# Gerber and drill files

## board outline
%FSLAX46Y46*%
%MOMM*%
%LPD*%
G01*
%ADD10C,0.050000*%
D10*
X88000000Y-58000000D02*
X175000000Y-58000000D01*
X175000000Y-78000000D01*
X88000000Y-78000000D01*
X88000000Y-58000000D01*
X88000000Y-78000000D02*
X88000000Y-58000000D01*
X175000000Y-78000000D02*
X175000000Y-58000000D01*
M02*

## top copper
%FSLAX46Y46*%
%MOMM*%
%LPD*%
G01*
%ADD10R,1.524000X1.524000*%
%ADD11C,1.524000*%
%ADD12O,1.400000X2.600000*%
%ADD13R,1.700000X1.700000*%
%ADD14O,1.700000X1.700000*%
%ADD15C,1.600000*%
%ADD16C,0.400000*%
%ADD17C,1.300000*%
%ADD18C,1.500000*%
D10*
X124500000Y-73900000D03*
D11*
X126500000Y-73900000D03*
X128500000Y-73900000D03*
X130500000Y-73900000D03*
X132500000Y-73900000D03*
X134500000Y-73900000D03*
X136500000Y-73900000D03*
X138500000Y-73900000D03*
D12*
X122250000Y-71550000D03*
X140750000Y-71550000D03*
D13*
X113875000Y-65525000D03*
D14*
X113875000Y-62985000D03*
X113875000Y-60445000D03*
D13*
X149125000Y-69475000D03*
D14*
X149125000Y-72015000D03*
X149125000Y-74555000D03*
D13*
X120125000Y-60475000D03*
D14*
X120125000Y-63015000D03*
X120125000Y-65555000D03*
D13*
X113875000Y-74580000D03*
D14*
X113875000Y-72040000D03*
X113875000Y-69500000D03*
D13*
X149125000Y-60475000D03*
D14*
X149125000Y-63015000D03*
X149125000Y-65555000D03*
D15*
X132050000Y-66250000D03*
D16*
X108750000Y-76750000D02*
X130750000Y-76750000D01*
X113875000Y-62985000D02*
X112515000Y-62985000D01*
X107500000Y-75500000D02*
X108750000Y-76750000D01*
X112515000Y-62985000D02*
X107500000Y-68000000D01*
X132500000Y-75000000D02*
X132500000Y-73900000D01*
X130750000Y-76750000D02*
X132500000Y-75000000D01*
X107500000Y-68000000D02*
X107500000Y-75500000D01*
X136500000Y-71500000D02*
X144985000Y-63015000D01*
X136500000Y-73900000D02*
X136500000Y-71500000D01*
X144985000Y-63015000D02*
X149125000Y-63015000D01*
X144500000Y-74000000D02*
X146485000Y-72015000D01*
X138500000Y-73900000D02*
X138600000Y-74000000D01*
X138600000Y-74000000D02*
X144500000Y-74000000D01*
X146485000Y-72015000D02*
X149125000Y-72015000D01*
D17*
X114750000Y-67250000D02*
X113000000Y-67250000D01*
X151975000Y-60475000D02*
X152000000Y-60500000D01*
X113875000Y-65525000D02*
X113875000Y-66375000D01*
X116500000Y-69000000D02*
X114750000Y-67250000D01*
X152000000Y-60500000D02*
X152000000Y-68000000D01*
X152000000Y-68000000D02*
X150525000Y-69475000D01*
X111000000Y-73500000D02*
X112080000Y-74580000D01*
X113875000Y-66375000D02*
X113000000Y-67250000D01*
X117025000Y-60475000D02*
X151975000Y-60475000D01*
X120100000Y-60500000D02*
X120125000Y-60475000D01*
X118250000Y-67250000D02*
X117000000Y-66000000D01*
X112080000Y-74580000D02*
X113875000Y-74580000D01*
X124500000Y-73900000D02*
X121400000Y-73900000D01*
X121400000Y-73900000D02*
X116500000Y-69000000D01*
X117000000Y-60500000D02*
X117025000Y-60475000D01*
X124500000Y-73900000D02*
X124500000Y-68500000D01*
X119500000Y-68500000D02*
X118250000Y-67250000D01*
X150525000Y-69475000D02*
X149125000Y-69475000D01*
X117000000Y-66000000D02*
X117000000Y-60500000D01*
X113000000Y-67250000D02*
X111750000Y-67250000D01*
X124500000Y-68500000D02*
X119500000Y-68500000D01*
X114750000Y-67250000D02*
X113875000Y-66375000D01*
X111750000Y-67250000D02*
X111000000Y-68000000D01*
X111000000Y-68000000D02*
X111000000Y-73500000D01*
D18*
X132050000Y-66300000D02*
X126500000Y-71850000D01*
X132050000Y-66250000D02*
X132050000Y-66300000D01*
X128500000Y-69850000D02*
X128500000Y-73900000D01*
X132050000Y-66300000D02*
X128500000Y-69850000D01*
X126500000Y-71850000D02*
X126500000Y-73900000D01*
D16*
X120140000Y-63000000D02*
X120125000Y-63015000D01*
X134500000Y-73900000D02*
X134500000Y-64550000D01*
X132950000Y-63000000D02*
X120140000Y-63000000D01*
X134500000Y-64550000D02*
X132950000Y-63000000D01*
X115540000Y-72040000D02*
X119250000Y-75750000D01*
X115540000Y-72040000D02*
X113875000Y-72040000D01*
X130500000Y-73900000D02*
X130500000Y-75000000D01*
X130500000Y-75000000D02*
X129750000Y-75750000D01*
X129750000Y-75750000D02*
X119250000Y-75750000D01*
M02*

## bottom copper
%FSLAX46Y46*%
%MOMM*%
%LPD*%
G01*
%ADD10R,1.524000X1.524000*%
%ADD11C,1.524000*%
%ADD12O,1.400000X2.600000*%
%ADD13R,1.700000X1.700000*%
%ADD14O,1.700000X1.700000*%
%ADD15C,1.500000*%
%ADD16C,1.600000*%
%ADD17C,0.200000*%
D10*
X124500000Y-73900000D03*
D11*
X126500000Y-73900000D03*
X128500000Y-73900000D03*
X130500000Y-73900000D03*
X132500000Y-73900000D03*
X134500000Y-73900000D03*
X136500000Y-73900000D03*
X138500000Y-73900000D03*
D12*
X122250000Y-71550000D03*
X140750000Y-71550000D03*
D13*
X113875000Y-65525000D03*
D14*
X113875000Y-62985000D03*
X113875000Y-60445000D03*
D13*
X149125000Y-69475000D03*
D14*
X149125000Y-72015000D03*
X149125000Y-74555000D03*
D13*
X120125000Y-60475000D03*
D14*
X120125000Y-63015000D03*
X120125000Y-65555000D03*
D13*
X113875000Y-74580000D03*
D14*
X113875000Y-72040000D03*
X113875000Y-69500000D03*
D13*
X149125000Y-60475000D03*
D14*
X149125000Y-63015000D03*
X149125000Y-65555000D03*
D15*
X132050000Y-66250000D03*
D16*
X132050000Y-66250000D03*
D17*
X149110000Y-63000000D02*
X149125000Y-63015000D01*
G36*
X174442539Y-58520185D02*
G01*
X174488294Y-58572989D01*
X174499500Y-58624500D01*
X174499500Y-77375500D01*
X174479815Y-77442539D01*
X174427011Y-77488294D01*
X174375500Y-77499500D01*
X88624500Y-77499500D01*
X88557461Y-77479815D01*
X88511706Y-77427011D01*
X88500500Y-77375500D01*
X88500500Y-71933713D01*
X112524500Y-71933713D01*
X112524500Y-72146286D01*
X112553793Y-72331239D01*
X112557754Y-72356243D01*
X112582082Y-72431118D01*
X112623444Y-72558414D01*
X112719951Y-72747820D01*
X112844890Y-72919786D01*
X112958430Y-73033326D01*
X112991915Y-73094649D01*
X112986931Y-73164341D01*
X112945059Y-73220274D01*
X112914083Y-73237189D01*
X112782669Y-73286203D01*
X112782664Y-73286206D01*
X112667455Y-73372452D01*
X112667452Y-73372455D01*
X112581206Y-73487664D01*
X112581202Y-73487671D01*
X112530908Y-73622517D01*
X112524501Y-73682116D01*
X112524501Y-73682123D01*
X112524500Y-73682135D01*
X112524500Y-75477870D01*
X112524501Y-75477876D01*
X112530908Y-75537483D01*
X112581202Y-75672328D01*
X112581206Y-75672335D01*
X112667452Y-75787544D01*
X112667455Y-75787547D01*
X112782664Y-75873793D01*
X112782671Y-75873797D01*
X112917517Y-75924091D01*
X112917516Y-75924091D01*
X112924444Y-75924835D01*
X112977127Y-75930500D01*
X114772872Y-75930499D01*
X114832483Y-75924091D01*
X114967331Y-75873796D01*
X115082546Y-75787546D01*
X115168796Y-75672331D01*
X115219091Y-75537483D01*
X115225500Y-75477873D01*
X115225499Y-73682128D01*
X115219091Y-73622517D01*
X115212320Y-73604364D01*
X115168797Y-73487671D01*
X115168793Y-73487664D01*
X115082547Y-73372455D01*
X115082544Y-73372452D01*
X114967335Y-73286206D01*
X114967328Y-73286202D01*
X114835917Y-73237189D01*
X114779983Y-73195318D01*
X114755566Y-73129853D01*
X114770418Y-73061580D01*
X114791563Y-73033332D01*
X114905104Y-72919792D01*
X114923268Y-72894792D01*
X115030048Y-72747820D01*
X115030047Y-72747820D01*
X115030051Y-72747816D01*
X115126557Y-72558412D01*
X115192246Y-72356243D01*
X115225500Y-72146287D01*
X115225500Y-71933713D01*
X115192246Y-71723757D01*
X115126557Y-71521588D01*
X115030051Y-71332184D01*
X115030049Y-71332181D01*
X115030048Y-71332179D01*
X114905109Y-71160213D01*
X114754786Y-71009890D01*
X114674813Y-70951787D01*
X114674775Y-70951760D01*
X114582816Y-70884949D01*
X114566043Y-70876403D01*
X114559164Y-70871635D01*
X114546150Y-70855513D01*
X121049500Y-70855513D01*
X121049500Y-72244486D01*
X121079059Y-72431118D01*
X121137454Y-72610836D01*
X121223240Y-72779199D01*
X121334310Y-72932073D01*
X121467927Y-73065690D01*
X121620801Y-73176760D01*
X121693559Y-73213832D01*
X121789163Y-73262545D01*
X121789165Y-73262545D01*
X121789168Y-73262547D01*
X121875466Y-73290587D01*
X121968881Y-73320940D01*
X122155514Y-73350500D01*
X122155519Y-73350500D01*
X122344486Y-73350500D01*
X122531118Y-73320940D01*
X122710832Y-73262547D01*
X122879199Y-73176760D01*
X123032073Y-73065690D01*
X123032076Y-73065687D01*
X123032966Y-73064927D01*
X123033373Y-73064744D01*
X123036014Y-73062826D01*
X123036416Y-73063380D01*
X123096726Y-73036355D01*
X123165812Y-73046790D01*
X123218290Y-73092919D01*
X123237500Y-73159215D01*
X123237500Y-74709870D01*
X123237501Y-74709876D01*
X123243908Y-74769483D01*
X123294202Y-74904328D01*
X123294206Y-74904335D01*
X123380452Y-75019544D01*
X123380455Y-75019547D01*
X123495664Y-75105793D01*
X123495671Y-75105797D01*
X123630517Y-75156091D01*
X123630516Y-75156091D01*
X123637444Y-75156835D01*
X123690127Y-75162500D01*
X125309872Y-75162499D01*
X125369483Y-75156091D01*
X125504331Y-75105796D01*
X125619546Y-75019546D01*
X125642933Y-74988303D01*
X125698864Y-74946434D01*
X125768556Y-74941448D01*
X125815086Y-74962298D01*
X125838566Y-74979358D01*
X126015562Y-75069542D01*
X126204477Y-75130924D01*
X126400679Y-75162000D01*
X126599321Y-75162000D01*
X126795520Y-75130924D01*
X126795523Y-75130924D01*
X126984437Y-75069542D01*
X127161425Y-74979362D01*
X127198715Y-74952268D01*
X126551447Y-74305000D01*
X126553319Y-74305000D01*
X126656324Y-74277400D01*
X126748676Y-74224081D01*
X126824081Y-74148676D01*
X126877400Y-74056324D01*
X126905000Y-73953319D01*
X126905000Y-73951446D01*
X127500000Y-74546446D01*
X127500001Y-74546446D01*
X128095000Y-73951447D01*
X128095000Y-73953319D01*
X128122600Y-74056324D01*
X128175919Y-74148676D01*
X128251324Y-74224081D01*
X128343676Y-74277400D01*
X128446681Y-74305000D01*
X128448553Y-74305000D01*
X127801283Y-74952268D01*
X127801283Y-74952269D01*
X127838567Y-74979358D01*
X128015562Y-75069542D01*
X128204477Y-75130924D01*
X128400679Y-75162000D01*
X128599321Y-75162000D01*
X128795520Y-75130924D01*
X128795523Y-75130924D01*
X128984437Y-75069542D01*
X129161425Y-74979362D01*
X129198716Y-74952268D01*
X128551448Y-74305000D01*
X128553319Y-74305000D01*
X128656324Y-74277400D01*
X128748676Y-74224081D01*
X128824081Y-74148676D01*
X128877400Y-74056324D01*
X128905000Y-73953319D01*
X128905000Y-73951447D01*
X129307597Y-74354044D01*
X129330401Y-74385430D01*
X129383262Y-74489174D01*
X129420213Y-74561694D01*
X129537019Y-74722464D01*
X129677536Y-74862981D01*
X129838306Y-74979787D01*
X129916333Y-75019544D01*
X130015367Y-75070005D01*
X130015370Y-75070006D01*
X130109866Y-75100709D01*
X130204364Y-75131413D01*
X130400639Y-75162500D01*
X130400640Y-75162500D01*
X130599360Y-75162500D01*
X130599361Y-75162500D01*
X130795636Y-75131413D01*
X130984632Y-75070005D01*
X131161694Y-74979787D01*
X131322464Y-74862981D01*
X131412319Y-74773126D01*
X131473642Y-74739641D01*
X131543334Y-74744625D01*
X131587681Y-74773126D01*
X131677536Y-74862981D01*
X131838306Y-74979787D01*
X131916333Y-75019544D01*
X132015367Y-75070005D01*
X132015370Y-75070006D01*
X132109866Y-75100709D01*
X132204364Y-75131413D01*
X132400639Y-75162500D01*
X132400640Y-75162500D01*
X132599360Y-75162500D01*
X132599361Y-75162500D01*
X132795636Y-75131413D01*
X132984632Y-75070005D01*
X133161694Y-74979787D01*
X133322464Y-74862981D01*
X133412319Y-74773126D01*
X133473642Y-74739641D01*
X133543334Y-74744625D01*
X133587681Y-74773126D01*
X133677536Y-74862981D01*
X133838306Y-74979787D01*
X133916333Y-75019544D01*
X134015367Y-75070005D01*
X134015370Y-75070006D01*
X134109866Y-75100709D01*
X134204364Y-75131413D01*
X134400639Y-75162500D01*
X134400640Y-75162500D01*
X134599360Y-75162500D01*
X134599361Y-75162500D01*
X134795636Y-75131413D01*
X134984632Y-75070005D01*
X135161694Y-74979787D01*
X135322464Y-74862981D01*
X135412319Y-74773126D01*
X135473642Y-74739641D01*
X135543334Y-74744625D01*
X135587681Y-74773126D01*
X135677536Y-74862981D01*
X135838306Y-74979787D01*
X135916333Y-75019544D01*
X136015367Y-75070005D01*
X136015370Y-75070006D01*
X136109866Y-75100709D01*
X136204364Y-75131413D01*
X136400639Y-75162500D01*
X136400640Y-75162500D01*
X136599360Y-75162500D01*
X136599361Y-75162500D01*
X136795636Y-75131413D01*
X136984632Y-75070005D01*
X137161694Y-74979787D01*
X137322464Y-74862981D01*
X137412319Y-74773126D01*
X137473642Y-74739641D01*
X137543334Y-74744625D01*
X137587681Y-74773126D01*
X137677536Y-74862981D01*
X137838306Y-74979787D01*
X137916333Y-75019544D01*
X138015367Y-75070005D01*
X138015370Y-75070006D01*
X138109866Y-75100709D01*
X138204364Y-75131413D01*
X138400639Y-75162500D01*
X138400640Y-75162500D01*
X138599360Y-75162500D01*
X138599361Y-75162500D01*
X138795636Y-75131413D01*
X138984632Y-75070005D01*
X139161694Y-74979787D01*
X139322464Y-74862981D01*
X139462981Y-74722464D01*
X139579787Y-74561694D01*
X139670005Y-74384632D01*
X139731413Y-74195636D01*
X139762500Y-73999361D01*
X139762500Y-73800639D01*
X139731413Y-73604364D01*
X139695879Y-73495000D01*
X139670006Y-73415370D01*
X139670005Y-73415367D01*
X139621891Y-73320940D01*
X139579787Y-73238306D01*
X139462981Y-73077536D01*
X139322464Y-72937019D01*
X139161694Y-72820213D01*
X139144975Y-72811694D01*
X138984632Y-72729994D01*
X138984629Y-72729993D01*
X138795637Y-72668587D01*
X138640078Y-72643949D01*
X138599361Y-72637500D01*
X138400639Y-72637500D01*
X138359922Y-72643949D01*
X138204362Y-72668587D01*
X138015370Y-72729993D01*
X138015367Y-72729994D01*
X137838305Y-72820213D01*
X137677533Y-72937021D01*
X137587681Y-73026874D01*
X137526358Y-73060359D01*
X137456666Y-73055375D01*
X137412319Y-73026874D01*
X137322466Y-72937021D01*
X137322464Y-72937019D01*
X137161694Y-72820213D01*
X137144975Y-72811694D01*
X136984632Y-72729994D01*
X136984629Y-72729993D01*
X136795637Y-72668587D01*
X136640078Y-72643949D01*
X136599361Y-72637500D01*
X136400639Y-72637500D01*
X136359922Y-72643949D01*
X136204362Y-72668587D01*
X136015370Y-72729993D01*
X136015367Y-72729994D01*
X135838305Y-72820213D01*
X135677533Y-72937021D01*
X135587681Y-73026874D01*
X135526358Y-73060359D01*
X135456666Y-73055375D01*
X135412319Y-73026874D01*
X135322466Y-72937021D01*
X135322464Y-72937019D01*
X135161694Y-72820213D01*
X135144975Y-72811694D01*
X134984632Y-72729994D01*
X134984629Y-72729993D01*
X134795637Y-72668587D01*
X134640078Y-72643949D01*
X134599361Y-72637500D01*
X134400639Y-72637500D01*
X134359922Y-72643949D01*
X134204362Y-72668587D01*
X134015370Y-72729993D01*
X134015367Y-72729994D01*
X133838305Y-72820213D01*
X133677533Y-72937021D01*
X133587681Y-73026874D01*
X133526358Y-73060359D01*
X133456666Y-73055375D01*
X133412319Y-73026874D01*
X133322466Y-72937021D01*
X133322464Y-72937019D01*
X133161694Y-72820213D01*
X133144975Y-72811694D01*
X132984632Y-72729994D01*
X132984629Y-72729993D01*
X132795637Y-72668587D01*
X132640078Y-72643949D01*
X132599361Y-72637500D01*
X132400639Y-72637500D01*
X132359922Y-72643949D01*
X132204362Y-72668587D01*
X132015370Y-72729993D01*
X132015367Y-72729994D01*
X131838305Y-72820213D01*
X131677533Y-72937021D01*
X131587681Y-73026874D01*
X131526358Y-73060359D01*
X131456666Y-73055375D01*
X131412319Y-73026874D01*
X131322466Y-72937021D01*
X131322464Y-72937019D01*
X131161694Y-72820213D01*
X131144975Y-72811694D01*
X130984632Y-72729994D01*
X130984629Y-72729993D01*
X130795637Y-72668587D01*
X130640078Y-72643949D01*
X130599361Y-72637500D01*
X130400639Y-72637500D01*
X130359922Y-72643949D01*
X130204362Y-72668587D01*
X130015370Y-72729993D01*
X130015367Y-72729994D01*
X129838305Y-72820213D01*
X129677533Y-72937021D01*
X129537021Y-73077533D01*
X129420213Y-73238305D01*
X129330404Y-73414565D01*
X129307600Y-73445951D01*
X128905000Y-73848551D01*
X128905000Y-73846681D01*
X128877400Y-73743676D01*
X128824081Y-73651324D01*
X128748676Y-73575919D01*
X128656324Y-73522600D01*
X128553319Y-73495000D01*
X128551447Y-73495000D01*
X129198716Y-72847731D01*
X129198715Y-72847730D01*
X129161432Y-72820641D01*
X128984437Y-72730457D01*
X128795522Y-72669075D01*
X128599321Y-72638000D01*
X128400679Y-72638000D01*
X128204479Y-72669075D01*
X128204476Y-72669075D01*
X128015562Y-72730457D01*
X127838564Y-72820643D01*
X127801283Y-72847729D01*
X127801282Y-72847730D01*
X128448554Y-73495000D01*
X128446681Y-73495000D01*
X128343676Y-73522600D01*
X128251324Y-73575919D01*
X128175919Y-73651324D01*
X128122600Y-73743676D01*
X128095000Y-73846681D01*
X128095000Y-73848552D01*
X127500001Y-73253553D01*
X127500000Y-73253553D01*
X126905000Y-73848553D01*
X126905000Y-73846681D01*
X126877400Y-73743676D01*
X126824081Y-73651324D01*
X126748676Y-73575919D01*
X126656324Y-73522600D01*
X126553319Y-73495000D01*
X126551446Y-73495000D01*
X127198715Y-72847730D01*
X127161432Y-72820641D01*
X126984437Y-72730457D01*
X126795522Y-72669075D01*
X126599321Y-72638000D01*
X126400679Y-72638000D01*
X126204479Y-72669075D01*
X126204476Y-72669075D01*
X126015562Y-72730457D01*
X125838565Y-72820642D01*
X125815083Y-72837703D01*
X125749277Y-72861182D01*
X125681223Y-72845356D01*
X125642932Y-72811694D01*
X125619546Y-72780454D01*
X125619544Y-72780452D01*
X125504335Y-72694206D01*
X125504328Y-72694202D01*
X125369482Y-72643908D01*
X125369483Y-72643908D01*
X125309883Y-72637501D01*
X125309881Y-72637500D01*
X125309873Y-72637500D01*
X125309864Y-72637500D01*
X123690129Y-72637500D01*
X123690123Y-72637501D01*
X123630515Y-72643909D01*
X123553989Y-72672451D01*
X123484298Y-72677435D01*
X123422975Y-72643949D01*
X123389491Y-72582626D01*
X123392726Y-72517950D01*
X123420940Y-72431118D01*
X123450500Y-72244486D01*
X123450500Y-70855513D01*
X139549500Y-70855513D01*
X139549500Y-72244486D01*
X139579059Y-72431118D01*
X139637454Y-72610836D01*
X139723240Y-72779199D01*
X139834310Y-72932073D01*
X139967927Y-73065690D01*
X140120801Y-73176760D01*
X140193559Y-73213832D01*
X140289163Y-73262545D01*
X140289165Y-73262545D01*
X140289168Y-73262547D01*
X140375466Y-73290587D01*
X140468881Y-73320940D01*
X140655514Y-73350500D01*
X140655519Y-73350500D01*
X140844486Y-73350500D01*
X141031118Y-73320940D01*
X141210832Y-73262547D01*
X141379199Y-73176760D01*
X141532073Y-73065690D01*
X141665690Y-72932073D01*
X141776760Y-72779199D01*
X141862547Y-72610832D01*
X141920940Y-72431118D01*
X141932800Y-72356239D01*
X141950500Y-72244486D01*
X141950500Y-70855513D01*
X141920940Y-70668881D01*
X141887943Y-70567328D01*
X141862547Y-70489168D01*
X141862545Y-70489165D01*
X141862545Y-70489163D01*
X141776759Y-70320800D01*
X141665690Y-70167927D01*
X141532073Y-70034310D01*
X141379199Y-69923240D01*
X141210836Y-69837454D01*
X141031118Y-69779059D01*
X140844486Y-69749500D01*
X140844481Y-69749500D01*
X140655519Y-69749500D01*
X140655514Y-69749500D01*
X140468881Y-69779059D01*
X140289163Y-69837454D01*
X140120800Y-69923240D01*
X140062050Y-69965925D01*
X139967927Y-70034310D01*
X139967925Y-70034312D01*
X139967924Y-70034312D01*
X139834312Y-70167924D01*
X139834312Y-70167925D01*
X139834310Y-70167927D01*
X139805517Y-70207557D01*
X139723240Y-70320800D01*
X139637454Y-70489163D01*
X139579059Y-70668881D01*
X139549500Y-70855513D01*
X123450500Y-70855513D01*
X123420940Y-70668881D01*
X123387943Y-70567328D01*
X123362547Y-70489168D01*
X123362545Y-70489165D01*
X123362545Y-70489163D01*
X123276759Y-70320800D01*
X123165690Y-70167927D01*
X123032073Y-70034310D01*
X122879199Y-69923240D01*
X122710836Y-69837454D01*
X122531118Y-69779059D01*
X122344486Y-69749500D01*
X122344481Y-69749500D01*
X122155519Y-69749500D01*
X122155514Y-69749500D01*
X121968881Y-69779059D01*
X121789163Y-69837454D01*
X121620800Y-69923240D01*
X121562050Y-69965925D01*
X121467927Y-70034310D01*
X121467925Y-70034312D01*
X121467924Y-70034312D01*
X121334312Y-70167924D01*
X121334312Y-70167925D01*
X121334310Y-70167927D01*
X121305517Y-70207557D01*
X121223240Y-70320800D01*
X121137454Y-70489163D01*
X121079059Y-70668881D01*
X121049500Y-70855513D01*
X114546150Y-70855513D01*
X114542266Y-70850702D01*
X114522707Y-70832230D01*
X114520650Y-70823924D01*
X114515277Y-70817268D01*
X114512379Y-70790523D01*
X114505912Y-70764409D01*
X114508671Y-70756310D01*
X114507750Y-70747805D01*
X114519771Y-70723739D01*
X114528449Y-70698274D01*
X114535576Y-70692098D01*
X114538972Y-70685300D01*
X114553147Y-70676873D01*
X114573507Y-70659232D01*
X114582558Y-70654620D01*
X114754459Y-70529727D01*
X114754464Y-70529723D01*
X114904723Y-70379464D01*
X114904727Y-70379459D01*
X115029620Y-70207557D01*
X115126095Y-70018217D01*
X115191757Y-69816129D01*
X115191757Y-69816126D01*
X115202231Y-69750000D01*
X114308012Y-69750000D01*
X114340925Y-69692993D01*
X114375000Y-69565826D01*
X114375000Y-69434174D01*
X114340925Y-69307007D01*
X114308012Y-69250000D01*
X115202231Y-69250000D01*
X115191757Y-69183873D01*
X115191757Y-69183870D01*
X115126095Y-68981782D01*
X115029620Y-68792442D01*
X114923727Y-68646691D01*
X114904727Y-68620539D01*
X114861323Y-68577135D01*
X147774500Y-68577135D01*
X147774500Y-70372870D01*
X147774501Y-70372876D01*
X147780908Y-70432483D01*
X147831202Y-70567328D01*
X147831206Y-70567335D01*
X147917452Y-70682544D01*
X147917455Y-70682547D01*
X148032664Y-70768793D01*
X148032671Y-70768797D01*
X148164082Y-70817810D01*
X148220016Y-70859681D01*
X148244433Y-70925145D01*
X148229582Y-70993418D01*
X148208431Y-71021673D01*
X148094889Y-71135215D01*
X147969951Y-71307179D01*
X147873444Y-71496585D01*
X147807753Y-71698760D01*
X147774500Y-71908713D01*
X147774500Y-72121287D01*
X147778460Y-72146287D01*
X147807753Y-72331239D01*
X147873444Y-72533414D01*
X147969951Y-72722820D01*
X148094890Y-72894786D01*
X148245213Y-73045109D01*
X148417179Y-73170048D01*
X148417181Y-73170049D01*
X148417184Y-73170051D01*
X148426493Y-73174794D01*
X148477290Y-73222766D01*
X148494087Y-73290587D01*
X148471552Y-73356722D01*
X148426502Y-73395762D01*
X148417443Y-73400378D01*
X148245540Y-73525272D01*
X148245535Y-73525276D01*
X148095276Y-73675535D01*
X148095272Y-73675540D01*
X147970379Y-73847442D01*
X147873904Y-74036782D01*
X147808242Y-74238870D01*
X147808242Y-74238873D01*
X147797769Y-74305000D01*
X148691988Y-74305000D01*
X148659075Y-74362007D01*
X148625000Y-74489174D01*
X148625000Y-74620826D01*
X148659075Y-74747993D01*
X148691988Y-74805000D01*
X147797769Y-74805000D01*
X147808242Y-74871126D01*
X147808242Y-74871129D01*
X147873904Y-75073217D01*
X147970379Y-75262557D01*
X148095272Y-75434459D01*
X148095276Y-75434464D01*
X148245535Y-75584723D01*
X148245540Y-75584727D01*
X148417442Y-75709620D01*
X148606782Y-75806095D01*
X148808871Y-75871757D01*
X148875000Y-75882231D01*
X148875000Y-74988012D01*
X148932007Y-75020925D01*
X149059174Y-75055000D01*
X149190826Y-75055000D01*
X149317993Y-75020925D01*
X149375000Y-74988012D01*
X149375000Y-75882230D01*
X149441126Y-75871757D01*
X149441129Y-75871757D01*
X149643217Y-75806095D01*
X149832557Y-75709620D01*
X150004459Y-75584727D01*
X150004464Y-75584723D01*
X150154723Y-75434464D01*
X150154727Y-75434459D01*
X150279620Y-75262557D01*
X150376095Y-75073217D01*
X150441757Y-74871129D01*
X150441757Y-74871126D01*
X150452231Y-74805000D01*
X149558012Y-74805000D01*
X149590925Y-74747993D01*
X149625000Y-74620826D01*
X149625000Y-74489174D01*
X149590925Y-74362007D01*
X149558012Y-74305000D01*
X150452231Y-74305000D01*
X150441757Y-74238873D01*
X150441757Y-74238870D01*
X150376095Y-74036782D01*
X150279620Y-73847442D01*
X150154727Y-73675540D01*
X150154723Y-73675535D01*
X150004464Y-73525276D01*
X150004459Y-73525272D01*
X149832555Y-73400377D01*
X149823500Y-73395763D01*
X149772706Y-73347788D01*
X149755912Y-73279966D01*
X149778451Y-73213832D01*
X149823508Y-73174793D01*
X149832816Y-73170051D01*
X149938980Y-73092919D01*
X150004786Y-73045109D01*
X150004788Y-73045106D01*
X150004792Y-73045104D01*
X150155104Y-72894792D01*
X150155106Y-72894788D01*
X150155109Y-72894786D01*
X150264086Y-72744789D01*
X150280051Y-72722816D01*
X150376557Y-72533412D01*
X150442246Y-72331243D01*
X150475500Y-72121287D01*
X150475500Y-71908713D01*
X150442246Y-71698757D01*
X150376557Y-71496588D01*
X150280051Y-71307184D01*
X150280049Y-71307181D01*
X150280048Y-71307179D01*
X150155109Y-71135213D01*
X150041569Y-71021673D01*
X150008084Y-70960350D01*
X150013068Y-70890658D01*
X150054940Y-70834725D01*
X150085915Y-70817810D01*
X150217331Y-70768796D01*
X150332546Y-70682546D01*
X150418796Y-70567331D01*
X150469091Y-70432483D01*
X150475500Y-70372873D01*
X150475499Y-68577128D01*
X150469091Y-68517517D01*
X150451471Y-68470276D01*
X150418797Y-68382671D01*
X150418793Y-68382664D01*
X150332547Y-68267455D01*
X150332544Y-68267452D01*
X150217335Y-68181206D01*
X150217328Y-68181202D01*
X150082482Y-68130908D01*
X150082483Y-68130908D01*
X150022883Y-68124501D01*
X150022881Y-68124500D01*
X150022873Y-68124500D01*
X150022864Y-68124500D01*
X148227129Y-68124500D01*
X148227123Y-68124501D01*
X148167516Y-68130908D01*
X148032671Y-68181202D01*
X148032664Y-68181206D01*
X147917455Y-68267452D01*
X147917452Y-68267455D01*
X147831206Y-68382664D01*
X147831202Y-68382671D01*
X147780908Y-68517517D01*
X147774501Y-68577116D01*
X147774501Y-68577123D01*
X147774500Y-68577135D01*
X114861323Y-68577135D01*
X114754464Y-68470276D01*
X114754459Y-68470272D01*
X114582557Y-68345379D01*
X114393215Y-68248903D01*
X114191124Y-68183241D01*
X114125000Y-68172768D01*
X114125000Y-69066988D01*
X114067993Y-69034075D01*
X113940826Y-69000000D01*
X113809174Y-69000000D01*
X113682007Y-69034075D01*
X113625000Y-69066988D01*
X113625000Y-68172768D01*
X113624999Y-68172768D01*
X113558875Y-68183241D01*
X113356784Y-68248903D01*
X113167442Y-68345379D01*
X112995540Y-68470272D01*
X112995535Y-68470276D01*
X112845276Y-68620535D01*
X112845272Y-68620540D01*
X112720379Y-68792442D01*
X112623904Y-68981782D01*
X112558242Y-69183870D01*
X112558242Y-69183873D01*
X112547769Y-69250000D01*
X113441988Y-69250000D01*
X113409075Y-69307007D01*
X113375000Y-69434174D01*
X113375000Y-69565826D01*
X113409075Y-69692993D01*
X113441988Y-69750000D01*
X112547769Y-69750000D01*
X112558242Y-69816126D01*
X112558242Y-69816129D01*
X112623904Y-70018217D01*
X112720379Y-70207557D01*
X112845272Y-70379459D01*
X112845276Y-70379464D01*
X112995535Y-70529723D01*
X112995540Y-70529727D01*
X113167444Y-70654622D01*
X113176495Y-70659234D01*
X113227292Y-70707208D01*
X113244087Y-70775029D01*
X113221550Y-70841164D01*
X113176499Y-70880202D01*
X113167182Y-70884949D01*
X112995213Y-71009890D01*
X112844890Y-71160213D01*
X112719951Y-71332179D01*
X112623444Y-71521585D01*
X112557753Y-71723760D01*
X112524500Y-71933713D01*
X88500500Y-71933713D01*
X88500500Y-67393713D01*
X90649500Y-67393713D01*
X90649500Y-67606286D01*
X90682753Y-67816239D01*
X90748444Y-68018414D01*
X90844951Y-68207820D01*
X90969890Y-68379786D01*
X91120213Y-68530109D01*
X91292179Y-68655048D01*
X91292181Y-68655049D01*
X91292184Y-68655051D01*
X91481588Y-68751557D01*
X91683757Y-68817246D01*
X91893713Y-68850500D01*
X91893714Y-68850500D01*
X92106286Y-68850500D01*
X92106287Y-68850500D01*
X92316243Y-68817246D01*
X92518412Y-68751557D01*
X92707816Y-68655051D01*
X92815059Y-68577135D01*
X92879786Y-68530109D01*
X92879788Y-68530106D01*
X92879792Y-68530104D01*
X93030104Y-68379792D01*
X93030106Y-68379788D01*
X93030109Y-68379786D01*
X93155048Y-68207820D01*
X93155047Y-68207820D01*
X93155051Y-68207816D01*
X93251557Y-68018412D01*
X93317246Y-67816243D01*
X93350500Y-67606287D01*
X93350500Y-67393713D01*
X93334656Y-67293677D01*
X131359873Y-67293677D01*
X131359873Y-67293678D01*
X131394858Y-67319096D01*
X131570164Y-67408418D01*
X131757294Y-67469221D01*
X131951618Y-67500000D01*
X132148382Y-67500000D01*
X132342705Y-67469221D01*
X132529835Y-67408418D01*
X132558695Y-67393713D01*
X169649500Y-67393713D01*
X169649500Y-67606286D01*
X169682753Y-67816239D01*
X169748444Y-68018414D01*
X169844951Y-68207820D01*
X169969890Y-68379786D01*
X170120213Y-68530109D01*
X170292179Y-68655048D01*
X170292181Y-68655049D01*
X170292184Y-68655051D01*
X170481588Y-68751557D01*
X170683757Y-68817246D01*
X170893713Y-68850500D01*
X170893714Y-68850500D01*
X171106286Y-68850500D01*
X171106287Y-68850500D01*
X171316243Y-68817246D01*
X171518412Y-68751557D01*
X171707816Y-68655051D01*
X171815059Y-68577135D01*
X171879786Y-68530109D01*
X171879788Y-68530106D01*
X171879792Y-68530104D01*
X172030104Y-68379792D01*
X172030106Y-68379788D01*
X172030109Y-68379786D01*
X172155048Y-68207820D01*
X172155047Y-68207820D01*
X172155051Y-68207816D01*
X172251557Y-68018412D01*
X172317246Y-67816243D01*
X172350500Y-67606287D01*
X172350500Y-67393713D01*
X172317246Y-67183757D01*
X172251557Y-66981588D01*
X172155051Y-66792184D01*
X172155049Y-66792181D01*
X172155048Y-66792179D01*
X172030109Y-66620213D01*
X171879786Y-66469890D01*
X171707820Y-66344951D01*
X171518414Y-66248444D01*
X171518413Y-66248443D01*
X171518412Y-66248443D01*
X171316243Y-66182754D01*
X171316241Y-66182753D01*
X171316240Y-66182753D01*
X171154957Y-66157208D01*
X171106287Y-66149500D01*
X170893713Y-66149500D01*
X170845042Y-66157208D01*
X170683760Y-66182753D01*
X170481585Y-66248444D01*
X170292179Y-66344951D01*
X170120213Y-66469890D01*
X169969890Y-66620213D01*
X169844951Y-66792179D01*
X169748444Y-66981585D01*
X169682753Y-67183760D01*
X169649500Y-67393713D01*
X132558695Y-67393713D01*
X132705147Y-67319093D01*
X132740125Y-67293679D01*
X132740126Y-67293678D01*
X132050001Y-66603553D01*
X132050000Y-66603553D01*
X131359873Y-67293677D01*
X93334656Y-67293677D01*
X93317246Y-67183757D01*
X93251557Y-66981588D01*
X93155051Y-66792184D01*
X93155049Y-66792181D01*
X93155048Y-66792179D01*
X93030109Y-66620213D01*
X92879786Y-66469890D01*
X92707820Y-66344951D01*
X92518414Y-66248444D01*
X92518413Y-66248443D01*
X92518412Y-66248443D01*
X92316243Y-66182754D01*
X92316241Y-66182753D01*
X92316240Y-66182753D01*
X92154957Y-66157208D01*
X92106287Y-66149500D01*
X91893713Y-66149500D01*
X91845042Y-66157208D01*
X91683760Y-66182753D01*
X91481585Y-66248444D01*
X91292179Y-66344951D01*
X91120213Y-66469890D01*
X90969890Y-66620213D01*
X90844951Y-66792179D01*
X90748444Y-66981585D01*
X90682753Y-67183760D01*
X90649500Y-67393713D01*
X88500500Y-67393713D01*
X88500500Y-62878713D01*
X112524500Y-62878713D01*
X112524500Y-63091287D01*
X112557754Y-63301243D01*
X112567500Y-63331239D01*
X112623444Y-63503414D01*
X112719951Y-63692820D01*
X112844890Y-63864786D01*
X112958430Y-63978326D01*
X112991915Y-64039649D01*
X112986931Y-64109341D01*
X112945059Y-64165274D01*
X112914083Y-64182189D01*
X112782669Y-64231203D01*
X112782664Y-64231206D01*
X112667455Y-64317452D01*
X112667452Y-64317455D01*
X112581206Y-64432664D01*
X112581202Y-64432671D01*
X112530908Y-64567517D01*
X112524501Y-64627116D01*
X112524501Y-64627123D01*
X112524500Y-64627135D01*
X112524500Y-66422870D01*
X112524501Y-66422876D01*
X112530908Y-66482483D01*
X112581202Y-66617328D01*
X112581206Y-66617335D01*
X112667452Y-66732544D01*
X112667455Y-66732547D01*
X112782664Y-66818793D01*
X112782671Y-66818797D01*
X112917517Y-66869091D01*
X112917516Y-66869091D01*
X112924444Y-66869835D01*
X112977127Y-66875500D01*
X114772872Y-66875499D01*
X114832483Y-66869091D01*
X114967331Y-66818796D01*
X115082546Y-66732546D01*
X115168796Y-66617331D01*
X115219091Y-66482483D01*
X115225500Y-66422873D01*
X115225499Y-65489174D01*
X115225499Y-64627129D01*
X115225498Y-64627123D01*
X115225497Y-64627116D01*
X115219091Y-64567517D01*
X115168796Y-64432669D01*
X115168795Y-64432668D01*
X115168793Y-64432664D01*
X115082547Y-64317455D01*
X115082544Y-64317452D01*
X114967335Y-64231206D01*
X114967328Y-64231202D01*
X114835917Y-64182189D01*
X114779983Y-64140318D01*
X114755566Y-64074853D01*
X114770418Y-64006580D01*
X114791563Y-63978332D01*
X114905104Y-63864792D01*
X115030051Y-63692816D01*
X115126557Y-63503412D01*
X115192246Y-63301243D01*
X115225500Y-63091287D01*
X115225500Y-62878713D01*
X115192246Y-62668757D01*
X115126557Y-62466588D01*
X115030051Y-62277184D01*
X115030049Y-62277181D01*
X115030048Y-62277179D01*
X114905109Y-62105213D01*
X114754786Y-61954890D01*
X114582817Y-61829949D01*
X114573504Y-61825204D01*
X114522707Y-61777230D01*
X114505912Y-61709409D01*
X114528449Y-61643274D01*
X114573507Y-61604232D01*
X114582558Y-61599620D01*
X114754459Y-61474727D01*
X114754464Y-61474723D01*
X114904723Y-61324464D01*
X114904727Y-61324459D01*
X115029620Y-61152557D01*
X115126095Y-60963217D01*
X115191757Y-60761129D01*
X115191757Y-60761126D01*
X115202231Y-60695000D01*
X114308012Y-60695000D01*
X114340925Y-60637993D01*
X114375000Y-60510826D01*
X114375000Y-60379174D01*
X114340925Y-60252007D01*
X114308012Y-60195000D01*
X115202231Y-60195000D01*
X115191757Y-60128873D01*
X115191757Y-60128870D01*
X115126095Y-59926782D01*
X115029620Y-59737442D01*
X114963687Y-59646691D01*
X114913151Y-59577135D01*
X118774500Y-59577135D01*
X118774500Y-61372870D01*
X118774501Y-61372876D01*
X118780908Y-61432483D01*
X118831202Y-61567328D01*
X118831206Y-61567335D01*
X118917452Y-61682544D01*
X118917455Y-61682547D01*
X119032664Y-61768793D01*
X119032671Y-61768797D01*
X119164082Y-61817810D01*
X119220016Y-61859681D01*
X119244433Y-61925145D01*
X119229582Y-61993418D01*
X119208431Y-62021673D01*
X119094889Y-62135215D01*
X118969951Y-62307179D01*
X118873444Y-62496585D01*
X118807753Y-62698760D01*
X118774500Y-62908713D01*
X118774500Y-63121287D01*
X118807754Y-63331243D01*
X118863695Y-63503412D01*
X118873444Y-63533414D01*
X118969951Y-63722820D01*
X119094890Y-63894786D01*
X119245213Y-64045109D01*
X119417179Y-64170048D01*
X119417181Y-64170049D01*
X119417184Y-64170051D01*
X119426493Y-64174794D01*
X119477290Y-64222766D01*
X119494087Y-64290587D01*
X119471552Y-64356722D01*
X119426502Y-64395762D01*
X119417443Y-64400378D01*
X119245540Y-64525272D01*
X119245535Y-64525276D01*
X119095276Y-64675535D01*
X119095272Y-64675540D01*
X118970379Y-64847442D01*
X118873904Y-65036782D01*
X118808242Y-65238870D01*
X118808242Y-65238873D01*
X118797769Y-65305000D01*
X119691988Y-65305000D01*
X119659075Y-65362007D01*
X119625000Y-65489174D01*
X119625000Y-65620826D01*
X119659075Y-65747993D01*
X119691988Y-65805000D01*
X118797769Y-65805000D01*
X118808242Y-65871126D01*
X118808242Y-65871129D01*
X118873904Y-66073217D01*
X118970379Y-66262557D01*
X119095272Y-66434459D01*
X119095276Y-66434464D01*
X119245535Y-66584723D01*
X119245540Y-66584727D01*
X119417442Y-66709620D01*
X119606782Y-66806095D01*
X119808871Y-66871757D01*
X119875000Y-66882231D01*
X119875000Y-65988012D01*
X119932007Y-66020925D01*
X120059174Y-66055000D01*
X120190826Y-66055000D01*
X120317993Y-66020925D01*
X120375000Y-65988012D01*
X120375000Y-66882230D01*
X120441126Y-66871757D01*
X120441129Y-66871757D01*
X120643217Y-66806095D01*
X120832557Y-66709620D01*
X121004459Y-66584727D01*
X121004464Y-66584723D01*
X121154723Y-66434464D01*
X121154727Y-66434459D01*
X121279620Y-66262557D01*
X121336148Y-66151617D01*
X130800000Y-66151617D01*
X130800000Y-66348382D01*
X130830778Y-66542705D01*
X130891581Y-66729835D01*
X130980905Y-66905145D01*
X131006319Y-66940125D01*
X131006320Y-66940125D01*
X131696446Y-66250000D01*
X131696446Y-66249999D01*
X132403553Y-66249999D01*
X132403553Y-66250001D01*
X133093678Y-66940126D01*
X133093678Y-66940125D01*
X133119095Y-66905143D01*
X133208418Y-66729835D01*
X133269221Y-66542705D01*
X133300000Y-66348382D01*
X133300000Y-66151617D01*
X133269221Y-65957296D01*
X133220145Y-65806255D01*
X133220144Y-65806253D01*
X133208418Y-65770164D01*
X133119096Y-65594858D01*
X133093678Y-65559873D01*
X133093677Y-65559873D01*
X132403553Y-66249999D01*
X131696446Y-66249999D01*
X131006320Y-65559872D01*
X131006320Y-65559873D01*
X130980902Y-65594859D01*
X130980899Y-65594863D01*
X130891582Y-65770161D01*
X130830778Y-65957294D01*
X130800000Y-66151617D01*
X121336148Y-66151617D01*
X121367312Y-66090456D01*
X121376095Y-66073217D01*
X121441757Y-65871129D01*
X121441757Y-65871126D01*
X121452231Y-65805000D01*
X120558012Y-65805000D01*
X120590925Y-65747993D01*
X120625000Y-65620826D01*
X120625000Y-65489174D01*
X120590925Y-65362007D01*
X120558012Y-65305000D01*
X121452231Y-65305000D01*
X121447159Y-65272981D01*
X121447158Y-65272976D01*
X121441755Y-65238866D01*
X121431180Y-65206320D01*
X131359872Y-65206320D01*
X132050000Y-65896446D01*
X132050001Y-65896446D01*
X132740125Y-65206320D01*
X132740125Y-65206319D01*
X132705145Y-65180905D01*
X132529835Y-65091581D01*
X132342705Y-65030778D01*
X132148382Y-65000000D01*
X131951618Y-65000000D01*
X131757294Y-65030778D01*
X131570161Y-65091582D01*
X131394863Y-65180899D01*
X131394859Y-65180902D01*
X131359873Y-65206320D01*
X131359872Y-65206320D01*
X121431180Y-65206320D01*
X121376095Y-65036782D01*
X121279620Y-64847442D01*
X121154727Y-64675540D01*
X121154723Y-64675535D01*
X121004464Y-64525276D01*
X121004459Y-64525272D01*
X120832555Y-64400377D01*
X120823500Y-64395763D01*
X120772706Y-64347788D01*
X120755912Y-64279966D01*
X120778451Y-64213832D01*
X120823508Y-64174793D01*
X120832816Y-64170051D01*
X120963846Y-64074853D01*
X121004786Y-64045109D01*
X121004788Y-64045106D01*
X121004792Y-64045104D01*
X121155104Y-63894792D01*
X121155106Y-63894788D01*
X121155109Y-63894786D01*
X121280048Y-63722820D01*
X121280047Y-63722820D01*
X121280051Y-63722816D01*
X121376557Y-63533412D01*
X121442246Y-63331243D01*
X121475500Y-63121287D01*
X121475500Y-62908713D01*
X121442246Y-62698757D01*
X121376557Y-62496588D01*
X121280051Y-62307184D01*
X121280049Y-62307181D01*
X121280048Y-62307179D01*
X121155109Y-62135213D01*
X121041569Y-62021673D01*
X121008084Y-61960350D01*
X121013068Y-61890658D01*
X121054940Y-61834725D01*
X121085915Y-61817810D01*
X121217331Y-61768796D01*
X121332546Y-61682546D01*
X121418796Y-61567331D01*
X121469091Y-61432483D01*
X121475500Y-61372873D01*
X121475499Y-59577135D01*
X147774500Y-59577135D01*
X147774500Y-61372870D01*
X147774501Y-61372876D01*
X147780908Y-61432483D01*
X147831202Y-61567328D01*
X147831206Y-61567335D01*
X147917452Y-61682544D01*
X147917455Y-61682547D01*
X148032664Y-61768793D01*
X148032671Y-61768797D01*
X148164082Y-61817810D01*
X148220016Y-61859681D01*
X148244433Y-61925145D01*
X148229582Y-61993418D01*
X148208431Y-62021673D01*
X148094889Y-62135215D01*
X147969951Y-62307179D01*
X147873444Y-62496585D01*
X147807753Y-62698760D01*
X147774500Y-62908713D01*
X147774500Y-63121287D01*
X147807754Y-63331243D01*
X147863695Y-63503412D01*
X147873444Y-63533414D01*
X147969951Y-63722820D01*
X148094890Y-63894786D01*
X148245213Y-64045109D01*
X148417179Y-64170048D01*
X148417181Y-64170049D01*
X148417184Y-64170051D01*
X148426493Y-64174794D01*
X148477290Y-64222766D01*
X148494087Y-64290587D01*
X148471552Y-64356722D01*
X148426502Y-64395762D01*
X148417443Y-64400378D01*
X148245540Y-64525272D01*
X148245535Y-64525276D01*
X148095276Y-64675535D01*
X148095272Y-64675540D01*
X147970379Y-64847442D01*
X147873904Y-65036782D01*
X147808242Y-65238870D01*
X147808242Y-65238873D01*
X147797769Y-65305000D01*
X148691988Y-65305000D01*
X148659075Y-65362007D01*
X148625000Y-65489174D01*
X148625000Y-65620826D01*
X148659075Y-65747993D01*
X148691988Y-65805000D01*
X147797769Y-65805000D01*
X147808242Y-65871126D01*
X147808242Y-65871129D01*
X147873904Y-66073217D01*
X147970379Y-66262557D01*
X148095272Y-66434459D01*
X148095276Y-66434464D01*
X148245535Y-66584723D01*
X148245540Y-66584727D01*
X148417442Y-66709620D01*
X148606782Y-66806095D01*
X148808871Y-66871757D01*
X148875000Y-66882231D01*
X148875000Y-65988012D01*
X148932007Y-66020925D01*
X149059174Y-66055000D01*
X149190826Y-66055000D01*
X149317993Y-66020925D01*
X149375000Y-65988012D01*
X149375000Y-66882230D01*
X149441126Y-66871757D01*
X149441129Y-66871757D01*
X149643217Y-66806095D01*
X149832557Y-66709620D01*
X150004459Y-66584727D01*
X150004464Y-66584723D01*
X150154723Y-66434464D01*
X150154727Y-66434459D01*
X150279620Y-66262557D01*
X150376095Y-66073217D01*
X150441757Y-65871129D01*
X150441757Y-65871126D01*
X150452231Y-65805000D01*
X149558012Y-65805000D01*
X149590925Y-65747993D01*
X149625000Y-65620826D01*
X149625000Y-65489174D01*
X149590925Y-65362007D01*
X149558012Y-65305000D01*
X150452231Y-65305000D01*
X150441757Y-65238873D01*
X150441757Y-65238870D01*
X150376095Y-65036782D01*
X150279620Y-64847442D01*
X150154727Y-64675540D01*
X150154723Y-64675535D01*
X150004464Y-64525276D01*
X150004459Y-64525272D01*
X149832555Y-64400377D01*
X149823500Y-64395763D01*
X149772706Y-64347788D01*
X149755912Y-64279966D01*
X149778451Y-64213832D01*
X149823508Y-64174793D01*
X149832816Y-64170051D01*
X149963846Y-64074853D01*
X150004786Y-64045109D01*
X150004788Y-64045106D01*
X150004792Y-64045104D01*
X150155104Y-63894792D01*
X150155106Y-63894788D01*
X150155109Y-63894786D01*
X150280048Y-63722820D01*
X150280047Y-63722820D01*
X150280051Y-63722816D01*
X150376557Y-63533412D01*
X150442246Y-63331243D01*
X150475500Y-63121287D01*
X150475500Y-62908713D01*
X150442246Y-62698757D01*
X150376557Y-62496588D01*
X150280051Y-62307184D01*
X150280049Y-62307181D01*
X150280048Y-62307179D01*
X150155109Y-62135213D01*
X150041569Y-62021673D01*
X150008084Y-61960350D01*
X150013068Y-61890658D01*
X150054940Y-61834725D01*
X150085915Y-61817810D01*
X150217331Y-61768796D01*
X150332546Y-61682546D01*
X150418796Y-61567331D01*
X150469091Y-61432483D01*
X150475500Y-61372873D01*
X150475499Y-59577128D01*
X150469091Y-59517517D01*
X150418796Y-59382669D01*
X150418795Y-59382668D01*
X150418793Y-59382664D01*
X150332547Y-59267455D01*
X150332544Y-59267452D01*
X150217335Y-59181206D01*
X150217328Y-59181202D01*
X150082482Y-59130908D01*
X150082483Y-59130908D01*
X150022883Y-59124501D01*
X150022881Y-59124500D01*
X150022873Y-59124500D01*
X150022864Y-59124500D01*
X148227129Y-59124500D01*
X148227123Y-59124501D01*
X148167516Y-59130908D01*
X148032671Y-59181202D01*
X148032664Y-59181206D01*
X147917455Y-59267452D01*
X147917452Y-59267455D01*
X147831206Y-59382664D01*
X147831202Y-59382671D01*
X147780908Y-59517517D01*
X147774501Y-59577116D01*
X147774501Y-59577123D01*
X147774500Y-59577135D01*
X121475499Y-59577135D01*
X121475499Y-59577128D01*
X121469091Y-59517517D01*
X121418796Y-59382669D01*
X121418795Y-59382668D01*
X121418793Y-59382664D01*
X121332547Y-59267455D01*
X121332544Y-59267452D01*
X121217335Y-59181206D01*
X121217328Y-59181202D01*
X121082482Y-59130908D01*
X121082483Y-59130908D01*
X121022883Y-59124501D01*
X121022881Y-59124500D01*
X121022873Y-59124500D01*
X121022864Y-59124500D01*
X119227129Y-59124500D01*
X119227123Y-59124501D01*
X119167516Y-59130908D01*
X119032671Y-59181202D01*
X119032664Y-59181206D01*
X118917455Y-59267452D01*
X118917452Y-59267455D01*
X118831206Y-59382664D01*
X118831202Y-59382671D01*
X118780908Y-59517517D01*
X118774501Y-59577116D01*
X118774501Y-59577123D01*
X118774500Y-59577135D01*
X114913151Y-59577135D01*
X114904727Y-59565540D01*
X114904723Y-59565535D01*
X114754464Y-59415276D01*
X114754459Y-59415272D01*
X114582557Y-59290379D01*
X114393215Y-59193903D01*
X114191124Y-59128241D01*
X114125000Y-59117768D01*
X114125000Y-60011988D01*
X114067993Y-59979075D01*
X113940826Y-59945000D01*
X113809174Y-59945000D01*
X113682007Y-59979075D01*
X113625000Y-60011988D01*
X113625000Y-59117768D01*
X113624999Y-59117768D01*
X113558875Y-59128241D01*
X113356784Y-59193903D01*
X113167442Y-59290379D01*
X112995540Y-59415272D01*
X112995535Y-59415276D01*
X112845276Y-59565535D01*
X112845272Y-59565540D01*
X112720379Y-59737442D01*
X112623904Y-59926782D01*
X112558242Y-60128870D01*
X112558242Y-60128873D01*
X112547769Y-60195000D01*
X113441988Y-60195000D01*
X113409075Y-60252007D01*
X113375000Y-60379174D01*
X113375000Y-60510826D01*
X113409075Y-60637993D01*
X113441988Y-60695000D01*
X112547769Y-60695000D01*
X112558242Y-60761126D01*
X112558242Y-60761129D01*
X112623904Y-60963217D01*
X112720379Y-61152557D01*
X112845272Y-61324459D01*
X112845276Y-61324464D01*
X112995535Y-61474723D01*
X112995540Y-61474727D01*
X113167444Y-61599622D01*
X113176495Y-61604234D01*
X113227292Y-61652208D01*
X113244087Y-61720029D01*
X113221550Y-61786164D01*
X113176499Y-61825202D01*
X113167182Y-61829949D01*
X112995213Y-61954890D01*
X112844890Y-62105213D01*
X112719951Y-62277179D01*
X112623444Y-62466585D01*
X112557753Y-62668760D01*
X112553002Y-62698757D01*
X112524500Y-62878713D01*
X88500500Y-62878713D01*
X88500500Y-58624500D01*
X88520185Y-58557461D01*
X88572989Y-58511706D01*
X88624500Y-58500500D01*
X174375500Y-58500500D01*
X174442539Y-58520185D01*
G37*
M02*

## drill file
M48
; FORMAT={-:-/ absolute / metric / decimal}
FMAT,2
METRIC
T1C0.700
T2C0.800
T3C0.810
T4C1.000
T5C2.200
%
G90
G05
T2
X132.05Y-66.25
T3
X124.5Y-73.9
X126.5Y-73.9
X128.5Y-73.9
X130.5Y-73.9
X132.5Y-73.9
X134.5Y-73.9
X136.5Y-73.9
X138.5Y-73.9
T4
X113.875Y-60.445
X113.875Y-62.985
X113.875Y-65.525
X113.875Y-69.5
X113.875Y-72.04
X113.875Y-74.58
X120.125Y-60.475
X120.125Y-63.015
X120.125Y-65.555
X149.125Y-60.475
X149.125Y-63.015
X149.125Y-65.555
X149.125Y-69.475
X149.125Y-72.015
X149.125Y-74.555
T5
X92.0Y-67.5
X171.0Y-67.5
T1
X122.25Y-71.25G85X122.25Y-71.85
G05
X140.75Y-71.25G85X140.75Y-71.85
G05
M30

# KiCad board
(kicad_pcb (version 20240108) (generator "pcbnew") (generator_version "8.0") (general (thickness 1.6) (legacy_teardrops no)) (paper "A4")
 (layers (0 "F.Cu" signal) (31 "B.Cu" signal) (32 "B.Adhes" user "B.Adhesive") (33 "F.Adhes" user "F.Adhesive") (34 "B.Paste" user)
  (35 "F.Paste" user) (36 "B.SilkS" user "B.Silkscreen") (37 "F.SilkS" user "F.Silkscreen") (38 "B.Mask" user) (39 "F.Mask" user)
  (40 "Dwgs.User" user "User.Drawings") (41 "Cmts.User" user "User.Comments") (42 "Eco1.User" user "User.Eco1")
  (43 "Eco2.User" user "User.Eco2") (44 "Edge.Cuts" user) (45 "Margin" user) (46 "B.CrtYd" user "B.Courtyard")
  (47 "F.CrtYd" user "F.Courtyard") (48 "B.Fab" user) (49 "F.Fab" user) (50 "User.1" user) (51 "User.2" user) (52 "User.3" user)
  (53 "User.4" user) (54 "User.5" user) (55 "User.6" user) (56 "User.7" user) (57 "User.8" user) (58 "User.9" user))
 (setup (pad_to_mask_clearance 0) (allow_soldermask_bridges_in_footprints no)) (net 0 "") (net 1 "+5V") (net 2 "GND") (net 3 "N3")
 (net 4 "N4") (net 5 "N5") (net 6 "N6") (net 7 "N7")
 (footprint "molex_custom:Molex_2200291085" (layer "F.Cu") (at 132.5 77.9)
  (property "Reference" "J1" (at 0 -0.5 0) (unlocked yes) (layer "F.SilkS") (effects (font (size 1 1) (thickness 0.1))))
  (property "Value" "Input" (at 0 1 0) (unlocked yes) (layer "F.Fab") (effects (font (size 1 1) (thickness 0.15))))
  (pad "1" thru_hole rect (at -8 -4 90) (size 1.524 1.524) (drill 0.81) (layers "*.Cu" "*.Mask") (remove_unused_layers no) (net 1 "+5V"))
  (pad "2" thru_hole circle (at -6 -4 90) (size 1.524 1.524) (drill 0.81) (layers "*.Cu" "*.Mask") (remove_unused_layers no) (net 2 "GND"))
  (pad "3" thru_hole circle (at -4 -4 90) (size 1.524 1.524) (drill 0.81) (layers "*.Cu" "*.Mask") (remove_unused_layers no) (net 2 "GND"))
  (pad "4" thru_hole circle (at -2 -4 90) (size 1.524 1.524) (drill 0.81) (layers "*.Cu" "*.Mask") (remove_unused_layers no) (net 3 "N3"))
  (pad "5" thru_hole circle (at 0 -4 90) (size 1.524 1.524) (drill 0.81) (layers "*.Cu" "*.Mask") (remove_unused_layers no) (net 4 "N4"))
  (pad "6" thru_hole circle (at 2 -4 90) (size 1.524 1.524) (drill 0.81) (layers "*.Cu" "*.Mask") (remove_unused_layers no) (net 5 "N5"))
  (pad "7" thru_hole circle (at 4 -4 90) (size 1.524 1.524) (drill 0.81) (layers "*.Cu" "*.Mask") (remove_unused_layers no) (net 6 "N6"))
  (pad "8" thru_hole circle (at 6 -4 90) (size 1.524 1.524) (drill 0.81) (layers "*.Cu" "*.Mask") (remove_unused_layers no) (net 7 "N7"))
  (pad "9" thru_hole oval (at -10.25 -6.35 270) (size 2.6 1.4) (drill oval 1.3 0.7) (layers "*.Cu" "*.Mask") (remove_unused_layers no))
  (pad "9" thru_hole oval (at 8.25 -6.35 270) (size 2.6 1.4) (drill oval 1.3 0.7) (layers "*.Cu" "*.Mask") (remove_unused_layers no)))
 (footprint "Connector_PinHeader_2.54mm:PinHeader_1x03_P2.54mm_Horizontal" (layer "F.Cu") (at 113.875 65.525 180)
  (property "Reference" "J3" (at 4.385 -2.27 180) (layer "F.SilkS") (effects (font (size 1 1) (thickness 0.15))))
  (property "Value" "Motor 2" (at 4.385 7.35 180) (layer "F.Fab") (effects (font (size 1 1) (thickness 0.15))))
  (pad "1" thru_hole rect (at 0 0 180) (size 1.7 1.7) (drill 1) (layers "*.Cu" "*.Mask") (remove_unused_layers no) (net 1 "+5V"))
  (pad "2" thru_hole oval (at 0 2.54 180) (size 1.7 1.7) (drill 1) (layers "*.Cu" "*.Mask") (remove_unused_layers no) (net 4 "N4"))
  (pad "3" thru_hole oval (at 0 5.08 180) (size 1.7 1.7) (drill 1) (layers "*.Cu" "*.Mask") (remove_unused_layers no) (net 2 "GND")))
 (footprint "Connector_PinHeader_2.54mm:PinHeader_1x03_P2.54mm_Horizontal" (layer "F.Cu") (at 149.125 69.475)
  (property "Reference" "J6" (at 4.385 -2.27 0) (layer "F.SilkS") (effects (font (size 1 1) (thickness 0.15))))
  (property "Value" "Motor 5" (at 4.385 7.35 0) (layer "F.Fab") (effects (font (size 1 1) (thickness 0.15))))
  (pad "1" thru_hole rect (at 0 0) (size 1.7 1.7) (drill 1) (layers "*.Cu" "*.Mask") (remove_unused_layers no) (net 1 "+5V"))
  (pad "2" thru_hole oval (at 0 2.54) (size 1.7 1.7) (drill 1) (layers "*.Cu" "*.Mask") (remove_unused_layers no) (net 7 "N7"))
  (pad "3" thru_hole oval (at 0 5.08) (size 1.7 1.7) (drill 1) (layers "*.Cu" "*.Mask") (remove_unused_layers no) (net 2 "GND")))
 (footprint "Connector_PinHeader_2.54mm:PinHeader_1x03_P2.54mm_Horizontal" (layer "F.Cu") (at 120.125 60.475)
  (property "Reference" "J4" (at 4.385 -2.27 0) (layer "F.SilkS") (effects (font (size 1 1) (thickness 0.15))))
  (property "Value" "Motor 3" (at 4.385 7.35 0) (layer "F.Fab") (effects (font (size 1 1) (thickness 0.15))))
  (pad "1" thru_hole rect (at 0 0) (size 1.7 1.7) (drill 1) (layers "*.Cu" "*.Mask") (remove_unused_layers no) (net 1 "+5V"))
  (pad "2" thru_hole oval (at 0 2.54) (size 1.7 1.7) (drill 1) (layers "*.Cu" "*.Mask") (remove_unused_layers no) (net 5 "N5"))
  (pad "3" thru_hole oval (at 0 5.08) (size 1.7 1.7) (drill 1) (layers "*.Cu" "*.Mask") (remove_unused_layers no) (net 2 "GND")))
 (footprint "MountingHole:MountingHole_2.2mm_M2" (layer "F.Cu") (at 171 67.5)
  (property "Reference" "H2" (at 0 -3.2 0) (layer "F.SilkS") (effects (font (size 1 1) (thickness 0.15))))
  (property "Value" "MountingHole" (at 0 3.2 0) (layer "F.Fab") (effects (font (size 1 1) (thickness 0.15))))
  (pad "" np_thru_hole circle (at 0 0) (size 2.2 2.2) (drill 2.2) (layers "*.Cu" "*.Mask")))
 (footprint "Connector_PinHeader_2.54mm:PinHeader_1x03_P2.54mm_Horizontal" (layer "F.Cu") (at 113.875 74.58 180)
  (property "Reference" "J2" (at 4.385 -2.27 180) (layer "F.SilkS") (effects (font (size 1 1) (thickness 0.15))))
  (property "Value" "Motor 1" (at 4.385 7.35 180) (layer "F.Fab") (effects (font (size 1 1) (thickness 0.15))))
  (pad "1" thru_hole rect (at 0 0 180) (size 1.7 1.7) (drill 1) (layers "*.Cu" "*.Mask") (remove_unused_layers no) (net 1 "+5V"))
  (pad "2" thru_hole oval (at 0 2.54 180) (size 1.7 1.7) (drill 1) (layers "*.Cu" "*.Mask") (remove_unused_layers no) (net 3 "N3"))
  (pad "3" thru_hole oval (at 0 5.08 180) (size 1.7 1.7) (drill 1) (layers "*.Cu" "*.Mask") (remove_unused_layers no) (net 2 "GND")))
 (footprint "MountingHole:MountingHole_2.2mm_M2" (layer "F.Cu") (at 92 67.5)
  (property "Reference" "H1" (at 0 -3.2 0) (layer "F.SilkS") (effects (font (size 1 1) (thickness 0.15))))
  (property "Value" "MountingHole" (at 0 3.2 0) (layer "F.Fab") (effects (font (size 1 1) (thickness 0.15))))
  (pad "" np_thru_hole circle (at 0 0) (size 2.2 2.2) (drill 2.2) (layers "*.Cu" "*.Mask")))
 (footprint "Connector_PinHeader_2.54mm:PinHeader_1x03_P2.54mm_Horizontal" (layer "F.Cu") (at 149.125 60.475)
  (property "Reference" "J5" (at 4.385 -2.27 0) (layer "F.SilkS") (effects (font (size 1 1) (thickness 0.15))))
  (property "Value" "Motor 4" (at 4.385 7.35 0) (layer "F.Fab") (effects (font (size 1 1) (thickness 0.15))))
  (pad "1" thru_hole rect (at 0 0) (size 1.7 1.7) (drill 1) (layers "*.Cu" "*.Mask") (remove_unused_layers no) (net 1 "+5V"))
  (pad "2" thru_hole oval (at 0 2.54) (size 1.7 1.7) (drill 1) (layers "*.Cu" "*.Mask") (remove_unused_layers no) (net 6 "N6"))
  (pad "3" thru_hole oval (at 0 5.08) (size 1.7 1.7) (drill 1) (layers "*.Cu" "*.Mask") (remove_unused_layers no) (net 2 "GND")))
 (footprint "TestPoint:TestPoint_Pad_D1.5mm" (layer "B.Cu") (at 132.05 66.25 180)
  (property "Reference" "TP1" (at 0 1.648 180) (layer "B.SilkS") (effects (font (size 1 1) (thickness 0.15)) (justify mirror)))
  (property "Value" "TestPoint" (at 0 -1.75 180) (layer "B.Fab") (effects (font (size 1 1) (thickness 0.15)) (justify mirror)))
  (pad "1" smd circle (at 0 0 180) (size 1.5 1.5) (layers "B.Cu" "B.Mask") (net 2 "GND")))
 (gr_rect (start 88 58) (end 175 78) (stroke (width 0.05) (type default)) (fill none) (layer "Edge.Cuts"))
 (gr_line (start 88 78) (end 88 58) (stroke (width 0.05) (type default)) (layer "Edge.Cuts"))
 (gr_line (start 175 78) (end 175 58) (stroke (width 0.05) (type default)) (layer "Edge.Cuts"))
 (segment (start 108.75 76.75) (end 130.75 76.75) (width 0.4) (layer "F.Cu") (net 4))
 (segment (start 113.875 62.985) (end 112.515 62.985) (width 0.4) (layer "F.Cu") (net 4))
 (segment (start 107.5 75.5) (end 108.75 76.75) (width 0.4) (layer "F.Cu") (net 4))
 (segment (start 112.515 62.985) (end 107.5 68) (width 0.4) (layer "F.Cu") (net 4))
 (segment (start 132.5 75) (end 132.5 73.9) (width 0.4) (layer "F.Cu") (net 4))
 (segment (start 130.75 76.75) (end 132.5 75) (width 0.4) (layer "F.Cu") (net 4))
 (segment (start 107.5 68) (end 107.5 75.5) (width 0.4) (layer "F.Cu") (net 4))
 (segment (start 136.5 71.5) (end 144.985 63.015) (width 0.4) (layer "F.Cu") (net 6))
 (segment (start 136.5 73.9) (end 136.5 71.5) (width 0.4) (layer "F.Cu") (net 6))
 (segment (start 144.985 63.015) (end 149.125 63.015) (width 0.4) (layer "F.Cu") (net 6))
 (segment (start 149.11 63) (end 149.125 63.015) (width 0.2) (layer "B.Cu") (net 6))
 (segment (start 144.5 74) (end 146.485 72.015) (width 0.4) (layer "F.Cu") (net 7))
 (segment (start 138.5 73.9) (end 138.6 74) (width 0.4) (layer "F.Cu") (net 7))
 (segment (start 138.6 74) (end 144.5 74) (width 0.4) (layer "F.Cu") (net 7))
 (segment (start 146.485 72.015) (end 149.125 72.015) (width 0.4) (layer "F.Cu") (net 7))
 (segment (start 114.75 67.25) (end 113 67.25) (width 1.3) (layer "F.Cu") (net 1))
 (segment (start 151.975 60.475) (end 152 60.5) (width 1.3) (layer "F.Cu") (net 1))
 (segment (start 113.875 65.525) (end 113.875 66.375) (width 1.3) (layer "F.Cu") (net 1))
 (segment (start 116.5 69) (end 114.75 67.25) (width 1.3) (layer "F.Cu") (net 1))
 (segment (start 152 60.5) (end 152 68) (width 1.3) (layer "F.Cu") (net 1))
 (segment (start 152 68) (end 150.525 69.475) (width 1.3) (layer "F.Cu") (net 1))
 (segment (start 111 73.5) (end 112.08 74.58) (width 1.3) (layer "F.Cu") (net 1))
 (segment (start 113.875 66.375) (end 113 67.25) (width 1.3) (layer "F.Cu") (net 1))
 (segment (start 117.025 60.475) (end 151.975 60.475) (width 1.3) (layer "F.Cu") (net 1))
 (segment (start 120.1 60.5) (end 120.125 60.475) (width 1.3) (layer "F.Cu") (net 1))
 (segment (start 118.25 67.25) (end 117 66) (width 1.3) (layer "F.Cu") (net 1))
 (segment (start 112.08 74.58) (end 113.875 74.58) (width 1.3) (layer "F.Cu") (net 1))
 (segment (start 124.5 73.9) (end 121.4 73.9) (width 1.3) (layer "F.Cu") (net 1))
 (segment (start 121.4 73.9) (end 116.5 69) (width 1.3) (layer "F.Cu") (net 1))
 (segment (start 117 60.5) (end 117.025 60.475) (width 1.3) (layer "F.Cu") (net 1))
 (segment (start 124.5 73.9) (end 124.5 68.5) (width 1.3) (layer "F.Cu") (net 1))
 (segment (start 119.5 68.5) (end 118.25 67.25) (width 1.3) (layer "F.Cu") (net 1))
 (segment (start 150.525 69.475) (end 149.125 69.475) (width 1.3) (layer "F.Cu") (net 1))
 (segment (start 117 66) (end 117 60.5) (width 1.3) (layer "F.Cu") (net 1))
 (segment (start 113 67.25) (end 111.75 67.25) (width 1.3) (layer "F.Cu") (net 1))
 (segment (start 124.5 68.5) (end 119.5 68.5) (width 1.3) (layer "F.Cu") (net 1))
 (segment (start 114.75 67.25) (end 113.875 66.375) (width 1.3) (layer "F.Cu") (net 1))
 (segment (start 111.75 67.25) (end 111 68) (width 1.3) (layer "F.Cu") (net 1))
 (segment (start 111 68) (end 111 73.5) (width 1.3) (layer "F.Cu") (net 1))
 (segment (start 132.05 66.3) (end 126.5 71.85) (width 1.5) (layer "F.Cu") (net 2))
 (segment (start 132.05 66.25) (end 132.05 66.3) (width 1.5) (layer "F.Cu") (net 2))
 (segment (start 128.5 69.85) (end 128.5 73.9) (width 1.5) (layer "F.Cu") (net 2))
 (segment (start 132.05 66.3) (end 128.5 69.85) (width 1.5) (layer "F.Cu") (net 2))
 (segment (start 126.5 71.85) (end 126.5 73.9) (width 1.5) (layer "F.Cu") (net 2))
 (via (at 132.05 66.25) (size 1.6) (drill 0.8) (layers "F.Cu" "B.Cu") (free yes) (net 2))
 (segment (start 120.14 63) (end 120.125 63.015) (width 0.4) (layer "F.Cu") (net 5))
 (segment (start 134.5 73.9) (end 134.5 64.55) (width 0.4) (layer "F.Cu") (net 5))
 (segment (start 132.95 63) (end 120.14 63) (width 0.4) (layer "F.Cu") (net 5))
 (segment (start 134.5 64.55) (end 132.95 63) (width 0.4) (layer "F.Cu") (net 5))
 (segment (start 115.54 72.04) (end 119.25 75.75) (width 0.4) (layer "F.Cu") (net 3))
 (segment (start 115.54 72.04) (end 113.875 72.04) (width 0.4) (layer "F.Cu") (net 3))
 (segment (start 130.5 73.9) (end 130.5 75) (width 0.4) (layer "F.Cu") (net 3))
 (segment (start 130.5 75) (end 129.75 75.75) (width 0.4) (layer "F.Cu") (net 3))
 (segment (start 129.75 75.75) (end 119.25 75.75) (width 0.4) (layer "F.Cu") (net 3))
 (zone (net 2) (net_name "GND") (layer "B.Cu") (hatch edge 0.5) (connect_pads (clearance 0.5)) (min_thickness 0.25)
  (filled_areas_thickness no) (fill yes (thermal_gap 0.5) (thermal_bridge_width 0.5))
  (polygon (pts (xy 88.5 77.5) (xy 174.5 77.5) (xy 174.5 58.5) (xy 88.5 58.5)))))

